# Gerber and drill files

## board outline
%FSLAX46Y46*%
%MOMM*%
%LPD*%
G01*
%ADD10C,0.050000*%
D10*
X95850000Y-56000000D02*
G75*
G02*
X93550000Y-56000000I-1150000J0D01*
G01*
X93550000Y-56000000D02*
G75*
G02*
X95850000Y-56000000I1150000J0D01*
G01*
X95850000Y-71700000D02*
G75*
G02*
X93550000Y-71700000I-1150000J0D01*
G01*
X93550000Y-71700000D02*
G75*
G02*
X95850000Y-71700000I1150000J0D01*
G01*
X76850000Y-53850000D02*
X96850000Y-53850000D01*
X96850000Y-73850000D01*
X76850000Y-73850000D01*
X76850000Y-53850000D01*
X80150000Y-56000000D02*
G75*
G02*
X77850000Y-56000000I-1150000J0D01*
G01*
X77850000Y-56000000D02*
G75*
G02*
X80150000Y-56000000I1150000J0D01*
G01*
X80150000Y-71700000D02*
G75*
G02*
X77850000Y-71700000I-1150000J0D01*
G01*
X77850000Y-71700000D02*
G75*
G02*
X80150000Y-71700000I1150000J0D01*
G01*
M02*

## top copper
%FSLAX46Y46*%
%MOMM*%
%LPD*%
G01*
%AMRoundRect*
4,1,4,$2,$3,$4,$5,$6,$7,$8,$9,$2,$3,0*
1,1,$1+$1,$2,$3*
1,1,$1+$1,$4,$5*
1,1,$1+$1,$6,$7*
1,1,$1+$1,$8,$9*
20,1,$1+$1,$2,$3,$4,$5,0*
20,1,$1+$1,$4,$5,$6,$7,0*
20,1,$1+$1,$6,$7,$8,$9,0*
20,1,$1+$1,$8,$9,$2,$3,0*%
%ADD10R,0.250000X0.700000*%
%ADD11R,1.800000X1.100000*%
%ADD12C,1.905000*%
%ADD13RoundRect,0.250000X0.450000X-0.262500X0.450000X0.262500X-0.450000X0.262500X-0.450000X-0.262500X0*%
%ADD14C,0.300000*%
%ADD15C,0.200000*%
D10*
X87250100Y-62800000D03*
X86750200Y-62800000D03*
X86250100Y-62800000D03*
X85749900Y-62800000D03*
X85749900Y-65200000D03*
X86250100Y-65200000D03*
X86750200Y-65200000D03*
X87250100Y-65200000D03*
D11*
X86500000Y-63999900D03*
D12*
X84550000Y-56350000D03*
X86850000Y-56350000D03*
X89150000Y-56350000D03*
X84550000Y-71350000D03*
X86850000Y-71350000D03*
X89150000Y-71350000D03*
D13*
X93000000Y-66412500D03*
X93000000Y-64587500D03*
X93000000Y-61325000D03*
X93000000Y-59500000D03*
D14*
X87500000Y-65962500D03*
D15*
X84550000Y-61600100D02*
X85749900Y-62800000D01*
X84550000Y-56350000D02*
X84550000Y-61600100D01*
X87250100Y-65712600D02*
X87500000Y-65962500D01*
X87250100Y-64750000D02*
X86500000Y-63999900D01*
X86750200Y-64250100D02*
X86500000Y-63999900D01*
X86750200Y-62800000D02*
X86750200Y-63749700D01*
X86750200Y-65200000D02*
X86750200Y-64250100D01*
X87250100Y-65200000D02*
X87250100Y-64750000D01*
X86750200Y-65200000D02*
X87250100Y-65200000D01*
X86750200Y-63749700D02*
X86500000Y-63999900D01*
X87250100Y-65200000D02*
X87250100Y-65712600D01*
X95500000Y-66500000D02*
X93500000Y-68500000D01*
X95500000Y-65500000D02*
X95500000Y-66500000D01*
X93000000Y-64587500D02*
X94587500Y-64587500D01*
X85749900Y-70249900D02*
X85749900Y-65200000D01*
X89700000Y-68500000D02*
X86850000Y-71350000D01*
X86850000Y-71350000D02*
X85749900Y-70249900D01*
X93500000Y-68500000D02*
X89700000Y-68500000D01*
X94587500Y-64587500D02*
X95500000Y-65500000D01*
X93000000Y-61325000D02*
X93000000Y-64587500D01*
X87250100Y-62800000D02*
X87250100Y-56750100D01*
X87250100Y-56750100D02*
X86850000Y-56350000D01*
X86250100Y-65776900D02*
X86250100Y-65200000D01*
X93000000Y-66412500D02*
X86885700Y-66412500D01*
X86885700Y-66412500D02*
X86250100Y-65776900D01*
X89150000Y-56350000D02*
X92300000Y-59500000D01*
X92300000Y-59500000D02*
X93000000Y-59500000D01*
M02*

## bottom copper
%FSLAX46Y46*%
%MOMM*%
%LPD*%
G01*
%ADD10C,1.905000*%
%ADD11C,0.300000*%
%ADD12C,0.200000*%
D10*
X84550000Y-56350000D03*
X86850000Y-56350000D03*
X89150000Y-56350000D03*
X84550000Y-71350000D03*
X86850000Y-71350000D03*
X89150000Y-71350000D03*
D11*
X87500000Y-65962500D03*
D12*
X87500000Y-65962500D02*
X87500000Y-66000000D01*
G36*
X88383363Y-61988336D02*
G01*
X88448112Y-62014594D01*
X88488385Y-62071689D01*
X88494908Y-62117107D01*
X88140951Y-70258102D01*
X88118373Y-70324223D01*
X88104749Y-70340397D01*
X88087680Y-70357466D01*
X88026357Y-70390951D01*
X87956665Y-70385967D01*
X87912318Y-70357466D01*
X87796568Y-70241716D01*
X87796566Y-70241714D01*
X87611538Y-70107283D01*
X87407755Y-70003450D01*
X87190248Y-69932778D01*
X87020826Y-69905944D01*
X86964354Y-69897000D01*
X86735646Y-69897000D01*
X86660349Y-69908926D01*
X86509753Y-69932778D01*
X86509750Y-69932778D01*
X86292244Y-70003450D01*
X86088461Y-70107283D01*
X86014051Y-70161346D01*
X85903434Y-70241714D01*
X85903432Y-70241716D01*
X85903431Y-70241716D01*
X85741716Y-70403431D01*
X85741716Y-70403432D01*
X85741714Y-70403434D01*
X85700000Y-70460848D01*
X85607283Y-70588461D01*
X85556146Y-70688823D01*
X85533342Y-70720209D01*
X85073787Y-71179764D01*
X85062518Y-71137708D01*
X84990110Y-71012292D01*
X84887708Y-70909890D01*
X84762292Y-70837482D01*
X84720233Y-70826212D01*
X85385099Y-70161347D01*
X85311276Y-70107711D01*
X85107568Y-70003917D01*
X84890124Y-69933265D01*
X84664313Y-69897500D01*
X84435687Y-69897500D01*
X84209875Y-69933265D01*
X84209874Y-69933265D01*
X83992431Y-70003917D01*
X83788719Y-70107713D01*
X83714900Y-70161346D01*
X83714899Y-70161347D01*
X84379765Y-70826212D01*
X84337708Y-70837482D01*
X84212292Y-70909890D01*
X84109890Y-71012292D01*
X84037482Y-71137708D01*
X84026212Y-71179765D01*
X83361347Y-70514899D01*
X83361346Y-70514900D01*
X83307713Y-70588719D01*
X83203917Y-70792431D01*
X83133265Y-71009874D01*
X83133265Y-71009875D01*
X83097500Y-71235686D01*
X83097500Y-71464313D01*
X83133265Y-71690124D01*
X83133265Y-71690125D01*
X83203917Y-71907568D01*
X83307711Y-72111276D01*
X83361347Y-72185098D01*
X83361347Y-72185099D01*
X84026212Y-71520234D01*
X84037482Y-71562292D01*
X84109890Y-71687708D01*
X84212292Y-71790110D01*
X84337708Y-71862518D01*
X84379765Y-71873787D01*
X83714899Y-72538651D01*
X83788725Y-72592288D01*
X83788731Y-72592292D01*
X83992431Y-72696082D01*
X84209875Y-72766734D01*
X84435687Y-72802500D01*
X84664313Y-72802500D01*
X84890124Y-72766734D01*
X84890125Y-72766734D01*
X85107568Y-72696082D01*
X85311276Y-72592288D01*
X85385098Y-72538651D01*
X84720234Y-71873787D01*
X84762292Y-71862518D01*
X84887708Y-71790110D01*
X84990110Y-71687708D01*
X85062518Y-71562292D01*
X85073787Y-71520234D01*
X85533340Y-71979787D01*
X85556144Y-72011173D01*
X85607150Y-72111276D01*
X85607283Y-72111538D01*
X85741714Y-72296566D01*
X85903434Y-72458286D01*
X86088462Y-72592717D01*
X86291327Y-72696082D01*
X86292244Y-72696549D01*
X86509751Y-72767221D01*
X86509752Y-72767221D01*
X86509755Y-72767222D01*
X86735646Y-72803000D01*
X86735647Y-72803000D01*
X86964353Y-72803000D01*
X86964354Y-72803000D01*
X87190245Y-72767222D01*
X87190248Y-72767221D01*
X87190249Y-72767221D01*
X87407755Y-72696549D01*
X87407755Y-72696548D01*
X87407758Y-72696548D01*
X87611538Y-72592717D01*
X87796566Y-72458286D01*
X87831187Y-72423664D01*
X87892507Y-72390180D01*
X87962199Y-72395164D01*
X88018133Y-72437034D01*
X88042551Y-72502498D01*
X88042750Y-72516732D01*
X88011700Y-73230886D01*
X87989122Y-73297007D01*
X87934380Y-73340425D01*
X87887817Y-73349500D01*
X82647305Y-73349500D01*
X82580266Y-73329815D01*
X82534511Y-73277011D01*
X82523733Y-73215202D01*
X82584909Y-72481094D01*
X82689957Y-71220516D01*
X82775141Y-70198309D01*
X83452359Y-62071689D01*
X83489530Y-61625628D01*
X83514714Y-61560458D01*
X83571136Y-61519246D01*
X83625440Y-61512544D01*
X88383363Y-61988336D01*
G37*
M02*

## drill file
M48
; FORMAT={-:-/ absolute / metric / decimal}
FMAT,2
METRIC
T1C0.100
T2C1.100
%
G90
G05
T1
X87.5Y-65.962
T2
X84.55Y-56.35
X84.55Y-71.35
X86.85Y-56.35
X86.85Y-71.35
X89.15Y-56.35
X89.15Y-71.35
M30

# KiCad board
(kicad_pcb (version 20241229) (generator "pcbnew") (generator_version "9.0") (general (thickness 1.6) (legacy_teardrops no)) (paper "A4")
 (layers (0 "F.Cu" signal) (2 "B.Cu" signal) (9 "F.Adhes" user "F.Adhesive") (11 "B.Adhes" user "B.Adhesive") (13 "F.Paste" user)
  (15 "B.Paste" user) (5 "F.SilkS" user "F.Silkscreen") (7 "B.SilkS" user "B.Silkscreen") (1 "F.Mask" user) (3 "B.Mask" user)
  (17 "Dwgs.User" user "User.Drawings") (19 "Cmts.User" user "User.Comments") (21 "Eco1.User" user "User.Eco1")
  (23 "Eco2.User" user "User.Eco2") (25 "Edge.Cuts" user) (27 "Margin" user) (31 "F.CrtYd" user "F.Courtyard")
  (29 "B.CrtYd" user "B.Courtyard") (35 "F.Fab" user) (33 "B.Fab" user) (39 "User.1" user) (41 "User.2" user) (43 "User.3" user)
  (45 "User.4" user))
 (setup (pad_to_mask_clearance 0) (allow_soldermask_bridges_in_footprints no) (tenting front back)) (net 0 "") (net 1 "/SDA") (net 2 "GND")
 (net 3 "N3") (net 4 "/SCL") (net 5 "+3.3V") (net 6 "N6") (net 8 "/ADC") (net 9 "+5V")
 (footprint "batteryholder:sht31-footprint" (layer "F.Cu") (at 86.5 64 180)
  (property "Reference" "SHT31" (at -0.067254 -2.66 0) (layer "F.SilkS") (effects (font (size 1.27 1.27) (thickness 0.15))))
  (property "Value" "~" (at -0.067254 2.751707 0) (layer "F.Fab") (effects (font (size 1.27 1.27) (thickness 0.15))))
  (pad "1" smd rect (at -0.7501 1.2 180) (size 0.25 0.7) (layers "F.Cu" "F.Mask" "F.Paste") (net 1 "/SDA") (solder_mask_margin 0.0508)
   (solder_paste_margin 0) (thermal_bridge_angle 0))
  (pad "2" smd rect (at -0.2502 1.2 180) (size 0.25 0.7) (layers "F.Cu" "F.Mask" "F.Paste") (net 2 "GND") (solder_mask_margin 0.0508)
   (solder_paste_margin 0) (thermal_bridge_angle 0))
  (pad "3" smd rect (at 0.2499 1.2 180) (size 0.25 0.7) (layers "F.Cu" "F.Mask" "F.Paste") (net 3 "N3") (solder_mask_margin 0.0508)
   (solder_paste_margin 0) (thermal_bridge_angle 0))
  (pad "4" smd rect (at 0.7501 1.2 180) (size 0.25 0.7) (layers "F.Cu" "F.Mask" "F.Paste") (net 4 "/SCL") (solder_mask_margin 0.0508)
   (solder_paste_margin 0) (thermal_bridge_angle 0))
  (pad "5" smd rect (at 0.7501 -1.2 180) (size 0.25 0.7) (layers "F.Cu" "F.Mask" "F.Paste") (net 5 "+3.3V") (solder_mask_margin 0.0508)
   (solder_paste_margin 0) (thermal_bridge_angle 0))
  (pad "6" smd rect (at 0.2499 -1.2 180) (size 0.25 0.7) (layers "F.Cu" "F.Mask" "F.Paste") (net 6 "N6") (solder_mask_margin 0.0508)
   (solder_paste_margin 0) (thermal_bridge_angle 0))
  (pad "7" smd rect (at -0.2502 -1.2 180) (size 0.25 0.7) (layers "F.Cu" "F.Mask" "F.Paste") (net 2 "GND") (solder_mask_margin 0.0508)
   (solder_paste_margin 0) (thermal_bridge_angle 0))
  (pad "8" smd rect (at -0.7501 -1.2 180) (size 0.25 0.7) (layers "F.Cu" "F.Mask" "F.Paste") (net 2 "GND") (solder_mask_margin 0.0508)
   (solder_paste_margin 0) (thermal_bridge_angle 0))
  (pad "9" smd rect (at 0 0.0001 180) (size 1.8 1.1) (layers "F.Cu" "F.Mask" "F.Paste") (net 2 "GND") (solder_mask_margin 0.0508)
   (solder_paste_margin 0) (thermal_bridge_angle 0))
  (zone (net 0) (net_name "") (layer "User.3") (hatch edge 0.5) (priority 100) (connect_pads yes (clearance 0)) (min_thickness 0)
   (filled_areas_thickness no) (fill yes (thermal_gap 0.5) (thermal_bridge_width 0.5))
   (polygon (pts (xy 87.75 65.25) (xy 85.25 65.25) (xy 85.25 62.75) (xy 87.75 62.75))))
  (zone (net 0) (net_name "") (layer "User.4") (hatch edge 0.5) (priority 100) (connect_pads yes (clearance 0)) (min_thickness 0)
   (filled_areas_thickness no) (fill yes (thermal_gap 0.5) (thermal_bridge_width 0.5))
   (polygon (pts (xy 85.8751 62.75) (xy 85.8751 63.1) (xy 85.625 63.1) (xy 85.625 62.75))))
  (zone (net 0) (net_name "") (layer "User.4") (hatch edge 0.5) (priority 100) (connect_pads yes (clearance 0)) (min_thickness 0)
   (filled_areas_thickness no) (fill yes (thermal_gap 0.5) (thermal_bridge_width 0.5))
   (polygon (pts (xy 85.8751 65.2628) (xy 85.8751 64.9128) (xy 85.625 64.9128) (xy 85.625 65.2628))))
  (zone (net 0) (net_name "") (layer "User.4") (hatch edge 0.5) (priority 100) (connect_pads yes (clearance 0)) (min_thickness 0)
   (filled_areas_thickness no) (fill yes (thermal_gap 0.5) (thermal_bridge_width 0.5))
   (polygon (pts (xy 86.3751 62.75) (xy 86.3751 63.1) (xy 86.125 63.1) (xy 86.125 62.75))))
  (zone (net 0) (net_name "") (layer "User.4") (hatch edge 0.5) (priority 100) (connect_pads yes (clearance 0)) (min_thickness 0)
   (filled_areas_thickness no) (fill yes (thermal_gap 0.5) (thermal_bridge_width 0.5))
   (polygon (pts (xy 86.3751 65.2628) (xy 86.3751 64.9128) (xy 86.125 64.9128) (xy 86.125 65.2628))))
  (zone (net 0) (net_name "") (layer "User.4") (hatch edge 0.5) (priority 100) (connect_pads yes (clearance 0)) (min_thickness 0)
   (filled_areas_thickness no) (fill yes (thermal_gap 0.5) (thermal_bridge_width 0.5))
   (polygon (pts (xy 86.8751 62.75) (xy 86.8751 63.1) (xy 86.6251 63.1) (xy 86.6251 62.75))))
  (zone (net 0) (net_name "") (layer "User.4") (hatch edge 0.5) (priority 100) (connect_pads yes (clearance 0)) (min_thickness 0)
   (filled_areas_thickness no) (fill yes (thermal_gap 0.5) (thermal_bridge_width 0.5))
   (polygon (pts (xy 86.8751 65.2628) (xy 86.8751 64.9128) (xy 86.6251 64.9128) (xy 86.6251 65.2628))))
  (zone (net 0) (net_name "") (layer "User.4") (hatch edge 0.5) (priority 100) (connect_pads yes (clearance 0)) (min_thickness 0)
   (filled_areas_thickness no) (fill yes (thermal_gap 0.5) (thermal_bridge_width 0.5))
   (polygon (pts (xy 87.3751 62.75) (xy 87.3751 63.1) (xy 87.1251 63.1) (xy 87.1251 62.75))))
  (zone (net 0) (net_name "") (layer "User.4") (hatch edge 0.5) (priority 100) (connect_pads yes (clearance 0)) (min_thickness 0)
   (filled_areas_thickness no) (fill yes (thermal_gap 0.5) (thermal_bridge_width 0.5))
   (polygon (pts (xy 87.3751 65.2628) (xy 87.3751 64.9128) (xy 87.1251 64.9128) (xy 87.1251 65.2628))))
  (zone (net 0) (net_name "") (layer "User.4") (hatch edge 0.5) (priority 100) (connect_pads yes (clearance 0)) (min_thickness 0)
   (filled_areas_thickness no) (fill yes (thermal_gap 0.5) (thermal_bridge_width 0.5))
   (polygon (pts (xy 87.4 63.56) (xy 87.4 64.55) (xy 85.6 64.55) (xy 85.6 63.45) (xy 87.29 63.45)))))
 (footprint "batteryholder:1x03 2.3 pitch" (layer "F.Cu") (at 84.25 56.35)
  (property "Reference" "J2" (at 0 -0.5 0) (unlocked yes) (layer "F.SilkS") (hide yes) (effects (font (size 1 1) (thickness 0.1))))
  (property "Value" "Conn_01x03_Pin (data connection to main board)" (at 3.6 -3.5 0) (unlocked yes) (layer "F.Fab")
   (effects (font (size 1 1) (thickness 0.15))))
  (pad "1" thru_hole circle (at 0.3 0) (size 1.905 1.905) (drill 1.1) (layers "*.Cu" "*.Mask") (remove_unused_layers no) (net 4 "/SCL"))
  (pad "2" thru_hole circle (at 2.6 0) (size 1.905 1.905) (drill 1.1) (layers "*.Cu" "*.Mask") (remove_unused_layers no) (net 1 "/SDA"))
  (pad "3" thru_hole circle (at 4.9 0) (size 1.905 1.905) (drill 1.1) (layers "*.Cu" "*.Mask") (remove_unused_layers no) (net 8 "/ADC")))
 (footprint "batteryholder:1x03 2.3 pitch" (layer "F.Cu") (at 84.75 71.35)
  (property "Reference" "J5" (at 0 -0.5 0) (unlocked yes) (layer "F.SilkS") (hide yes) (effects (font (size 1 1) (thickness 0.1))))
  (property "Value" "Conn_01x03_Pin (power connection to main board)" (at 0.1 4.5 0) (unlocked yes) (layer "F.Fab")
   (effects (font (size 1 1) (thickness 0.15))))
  (pad "1" thru_hole circle (at -0.2 0) (size 1.905 1.905) (drill 1.1) (layers "*.Cu" "*.Mask") (remove_unused_layers no) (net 2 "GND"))
  (pad "2" thru_hole circle (at 2.1 0) (size 1.905 1.905) (drill 1.1) (layers "*.Cu" "*.Mask") (remove_unused_layers no) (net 5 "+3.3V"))
  (pad "3" thru_hole circle (at 4.4 0) (size 1.905 1.905) (drill 1.1) (layers "*.Cu" "*.Mask") (remove_unused_layers no) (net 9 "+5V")))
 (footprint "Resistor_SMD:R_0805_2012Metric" (layer "F.Cu") (at 93 65.5 90)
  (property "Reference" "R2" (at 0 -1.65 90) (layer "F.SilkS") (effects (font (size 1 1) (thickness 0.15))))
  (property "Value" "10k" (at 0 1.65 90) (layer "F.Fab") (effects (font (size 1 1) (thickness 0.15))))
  (pad "1" smd roundrect (at -0.9125 0 90) (size 1.025 1.4) (layers "F.Cu" "F.Mask" "F.Paste") (roundrect_rratio 0.243902) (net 6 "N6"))
  (pad "2" smd roundrect (at 0.9125 0 90) (size 1.025 1.4) (layers "F.Cu" "F.Mask" "F.Paste") (roundrect_rratio 0.243902) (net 5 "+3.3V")))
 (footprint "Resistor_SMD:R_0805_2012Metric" (layer "F.Cu") (at 93 60.4125 90)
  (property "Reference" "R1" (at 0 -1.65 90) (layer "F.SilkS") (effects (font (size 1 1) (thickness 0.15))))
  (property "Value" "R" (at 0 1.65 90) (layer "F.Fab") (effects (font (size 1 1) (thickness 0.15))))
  (pad "1" smd roundrect (at -0.9125 0 90) (size 1.025 1.4) (layers "F.Cu" "F.Mask" "F.Paste") (roundrect_rratio 0.243902) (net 5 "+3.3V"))
  (pad "2" smd roundrect (at 0.9125 0 90) (size 1.025 1.4) (layers "F.Cu" "F.Mask" "F.Paste") (roundrect_rratio 0.243902) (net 8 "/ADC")))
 (gr_circle (center 94.7 56) (end 95.85 56) (stroke (width 0.05) (type solid)) (fill no) (layer "Edge.Cuts"))
 (gr_circle (center 94.7 71.7) (end 95.85 71.7) (stroke (width 0.05) (type solid)) (fill no) (layer "Edge.Cuts"))
 (gr_rect (start 76.85 53.85) (end 96.85 73.85) (stroke (width 0.05) (type solid)) (fill no) (layer "Edge.Cuts"))
 (gr_circle (center 79 56) (end 80.15 56) (stroke (width 0.05) (type solid)) (fill no) (layer "Edge.Cuts"))
 (gr_circle (center 79 71.7) (end 80.15 71.7) (stroke (width 0.05) (type solid)) (fill no) (layer "Edge.Cuts"))
 (segment (start 84.55 61.6001) (end 85.7499 62.8) (width 0.2) (layer "F.Cu") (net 4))
 (segment (start 84.55 56.35) (end 84.55 61.6001) (width 0.2) (layer "F.Cu") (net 4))
 (segment (start 87.2501 65.7126) (end 87.5 65.9625) (width 0.2) (layer "F.Cu") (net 2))
 (segment (start 87.2501 64.75) (end 86.5 63.9999) (width 0.2) (layer "F.Cu") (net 2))
 (segment (start 86.7502 64.2501) (end 86.5 63.9999) (width 0.2) (layer "F.Cu") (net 2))
 (segment (start 86.7502 62.8) (end 86.7502 63.7497) (width 0.2) (layer "F.Cu") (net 2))
 (segment (start 86.7502 65.2) (end 86.7502 64.2501) (width 0.2) (layer "F.Cu") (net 2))
 (segment (start 87.2501 65.2) (end 87.2501 64.75) (width 0.2) (layer "F.Cu") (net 2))
 (segment (start 86.7502 65.2) (end 87.2501 65.2) (width 0.2) (layer "F.Cu") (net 2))
 (segment (start 86.7502 63.7497) (end 86.5 63.9999) (width 0.2) (layer "F.Cu") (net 2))
 (segment (start 87.2501 65.2) (end 87.2501 65.7126) (width 0.2) (layer "F.Cu") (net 2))
 (via micro (at 87.5 65.9625) (size 0.3) (drill 0.1) (layers "F.Cu" "B.Cu") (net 2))
 (segment (start 87.5 65.9625) (end 87.5 66) (width 0.2) (layer "B.Cu") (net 2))
 (segment (start 95.5 66.5) (end 93.5 68.5) (width 0.2) (layer "F.Cu") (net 5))
 (segment (start 95.5 65.5) (end 95.5 66.5) (width 0.2) (layer "F.Cu") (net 5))
 (segment (start 93 64.5875) (end 94.5875 64.5875) (width 0.2) (layer "F.Cu") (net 5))
 (segment (start 85.7499 70.2499) (end 85.7499 65.2) (width 0.2) (layer "F.Cu") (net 5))
 (segment (start 89.7 68.5) (end 86.85 71.35) (width 0.2) (layer "F.Cu") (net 5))
 (segment (start 86.85 71.35) (end 85.7499 70.2499) (width 0.2) (layer "F.Cu") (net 5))
 (segment (start 93.5 68.5) (end 89.7 68.5) (width 0.2) (layer "F.Cu") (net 5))
 (segment (start 94.5875 64.5875) (end 95.5 65.5) (width 0.2) (layer "F.Cu") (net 5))
 (segment (start 93 61.325) (end 93 64.5875) (width 0.2) (layer "F.Cu") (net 5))
 (segment (start 87.2501 62.8) (end 87.2501 56.7501) (width 0.2) (layer "F.Cu") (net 1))
 (segment (start 87.2501 56.7501) (end 86.85 56.35) (width 0.2) (layer "F.Cu") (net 1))
 (segment (start 86.2501 65.7769) (end 86.2501 65.2) (width 0.2) (layer "F.Cu") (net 6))
 (segment (start 93 66.4125) (end 86.8857 66.4125) (width 0.2) (layer "F.Cu") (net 6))
 (segment (start 86.8857 66.4125) (end 86.2501 65.7769) (width 0.2) (layer "F.Cu") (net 6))
 (segment (start 89.15 56.35) (end 92.3 59.5) (width 0.2) (layer "F.Cu") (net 8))
 (segment (start 92.3 59.5) (end 93 59.5) (width 0.2) (layer "F.Cu") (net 8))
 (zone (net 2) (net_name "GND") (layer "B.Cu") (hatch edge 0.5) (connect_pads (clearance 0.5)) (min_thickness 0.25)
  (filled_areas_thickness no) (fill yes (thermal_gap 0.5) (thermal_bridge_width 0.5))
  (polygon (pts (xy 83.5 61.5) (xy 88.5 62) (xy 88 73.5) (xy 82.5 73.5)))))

